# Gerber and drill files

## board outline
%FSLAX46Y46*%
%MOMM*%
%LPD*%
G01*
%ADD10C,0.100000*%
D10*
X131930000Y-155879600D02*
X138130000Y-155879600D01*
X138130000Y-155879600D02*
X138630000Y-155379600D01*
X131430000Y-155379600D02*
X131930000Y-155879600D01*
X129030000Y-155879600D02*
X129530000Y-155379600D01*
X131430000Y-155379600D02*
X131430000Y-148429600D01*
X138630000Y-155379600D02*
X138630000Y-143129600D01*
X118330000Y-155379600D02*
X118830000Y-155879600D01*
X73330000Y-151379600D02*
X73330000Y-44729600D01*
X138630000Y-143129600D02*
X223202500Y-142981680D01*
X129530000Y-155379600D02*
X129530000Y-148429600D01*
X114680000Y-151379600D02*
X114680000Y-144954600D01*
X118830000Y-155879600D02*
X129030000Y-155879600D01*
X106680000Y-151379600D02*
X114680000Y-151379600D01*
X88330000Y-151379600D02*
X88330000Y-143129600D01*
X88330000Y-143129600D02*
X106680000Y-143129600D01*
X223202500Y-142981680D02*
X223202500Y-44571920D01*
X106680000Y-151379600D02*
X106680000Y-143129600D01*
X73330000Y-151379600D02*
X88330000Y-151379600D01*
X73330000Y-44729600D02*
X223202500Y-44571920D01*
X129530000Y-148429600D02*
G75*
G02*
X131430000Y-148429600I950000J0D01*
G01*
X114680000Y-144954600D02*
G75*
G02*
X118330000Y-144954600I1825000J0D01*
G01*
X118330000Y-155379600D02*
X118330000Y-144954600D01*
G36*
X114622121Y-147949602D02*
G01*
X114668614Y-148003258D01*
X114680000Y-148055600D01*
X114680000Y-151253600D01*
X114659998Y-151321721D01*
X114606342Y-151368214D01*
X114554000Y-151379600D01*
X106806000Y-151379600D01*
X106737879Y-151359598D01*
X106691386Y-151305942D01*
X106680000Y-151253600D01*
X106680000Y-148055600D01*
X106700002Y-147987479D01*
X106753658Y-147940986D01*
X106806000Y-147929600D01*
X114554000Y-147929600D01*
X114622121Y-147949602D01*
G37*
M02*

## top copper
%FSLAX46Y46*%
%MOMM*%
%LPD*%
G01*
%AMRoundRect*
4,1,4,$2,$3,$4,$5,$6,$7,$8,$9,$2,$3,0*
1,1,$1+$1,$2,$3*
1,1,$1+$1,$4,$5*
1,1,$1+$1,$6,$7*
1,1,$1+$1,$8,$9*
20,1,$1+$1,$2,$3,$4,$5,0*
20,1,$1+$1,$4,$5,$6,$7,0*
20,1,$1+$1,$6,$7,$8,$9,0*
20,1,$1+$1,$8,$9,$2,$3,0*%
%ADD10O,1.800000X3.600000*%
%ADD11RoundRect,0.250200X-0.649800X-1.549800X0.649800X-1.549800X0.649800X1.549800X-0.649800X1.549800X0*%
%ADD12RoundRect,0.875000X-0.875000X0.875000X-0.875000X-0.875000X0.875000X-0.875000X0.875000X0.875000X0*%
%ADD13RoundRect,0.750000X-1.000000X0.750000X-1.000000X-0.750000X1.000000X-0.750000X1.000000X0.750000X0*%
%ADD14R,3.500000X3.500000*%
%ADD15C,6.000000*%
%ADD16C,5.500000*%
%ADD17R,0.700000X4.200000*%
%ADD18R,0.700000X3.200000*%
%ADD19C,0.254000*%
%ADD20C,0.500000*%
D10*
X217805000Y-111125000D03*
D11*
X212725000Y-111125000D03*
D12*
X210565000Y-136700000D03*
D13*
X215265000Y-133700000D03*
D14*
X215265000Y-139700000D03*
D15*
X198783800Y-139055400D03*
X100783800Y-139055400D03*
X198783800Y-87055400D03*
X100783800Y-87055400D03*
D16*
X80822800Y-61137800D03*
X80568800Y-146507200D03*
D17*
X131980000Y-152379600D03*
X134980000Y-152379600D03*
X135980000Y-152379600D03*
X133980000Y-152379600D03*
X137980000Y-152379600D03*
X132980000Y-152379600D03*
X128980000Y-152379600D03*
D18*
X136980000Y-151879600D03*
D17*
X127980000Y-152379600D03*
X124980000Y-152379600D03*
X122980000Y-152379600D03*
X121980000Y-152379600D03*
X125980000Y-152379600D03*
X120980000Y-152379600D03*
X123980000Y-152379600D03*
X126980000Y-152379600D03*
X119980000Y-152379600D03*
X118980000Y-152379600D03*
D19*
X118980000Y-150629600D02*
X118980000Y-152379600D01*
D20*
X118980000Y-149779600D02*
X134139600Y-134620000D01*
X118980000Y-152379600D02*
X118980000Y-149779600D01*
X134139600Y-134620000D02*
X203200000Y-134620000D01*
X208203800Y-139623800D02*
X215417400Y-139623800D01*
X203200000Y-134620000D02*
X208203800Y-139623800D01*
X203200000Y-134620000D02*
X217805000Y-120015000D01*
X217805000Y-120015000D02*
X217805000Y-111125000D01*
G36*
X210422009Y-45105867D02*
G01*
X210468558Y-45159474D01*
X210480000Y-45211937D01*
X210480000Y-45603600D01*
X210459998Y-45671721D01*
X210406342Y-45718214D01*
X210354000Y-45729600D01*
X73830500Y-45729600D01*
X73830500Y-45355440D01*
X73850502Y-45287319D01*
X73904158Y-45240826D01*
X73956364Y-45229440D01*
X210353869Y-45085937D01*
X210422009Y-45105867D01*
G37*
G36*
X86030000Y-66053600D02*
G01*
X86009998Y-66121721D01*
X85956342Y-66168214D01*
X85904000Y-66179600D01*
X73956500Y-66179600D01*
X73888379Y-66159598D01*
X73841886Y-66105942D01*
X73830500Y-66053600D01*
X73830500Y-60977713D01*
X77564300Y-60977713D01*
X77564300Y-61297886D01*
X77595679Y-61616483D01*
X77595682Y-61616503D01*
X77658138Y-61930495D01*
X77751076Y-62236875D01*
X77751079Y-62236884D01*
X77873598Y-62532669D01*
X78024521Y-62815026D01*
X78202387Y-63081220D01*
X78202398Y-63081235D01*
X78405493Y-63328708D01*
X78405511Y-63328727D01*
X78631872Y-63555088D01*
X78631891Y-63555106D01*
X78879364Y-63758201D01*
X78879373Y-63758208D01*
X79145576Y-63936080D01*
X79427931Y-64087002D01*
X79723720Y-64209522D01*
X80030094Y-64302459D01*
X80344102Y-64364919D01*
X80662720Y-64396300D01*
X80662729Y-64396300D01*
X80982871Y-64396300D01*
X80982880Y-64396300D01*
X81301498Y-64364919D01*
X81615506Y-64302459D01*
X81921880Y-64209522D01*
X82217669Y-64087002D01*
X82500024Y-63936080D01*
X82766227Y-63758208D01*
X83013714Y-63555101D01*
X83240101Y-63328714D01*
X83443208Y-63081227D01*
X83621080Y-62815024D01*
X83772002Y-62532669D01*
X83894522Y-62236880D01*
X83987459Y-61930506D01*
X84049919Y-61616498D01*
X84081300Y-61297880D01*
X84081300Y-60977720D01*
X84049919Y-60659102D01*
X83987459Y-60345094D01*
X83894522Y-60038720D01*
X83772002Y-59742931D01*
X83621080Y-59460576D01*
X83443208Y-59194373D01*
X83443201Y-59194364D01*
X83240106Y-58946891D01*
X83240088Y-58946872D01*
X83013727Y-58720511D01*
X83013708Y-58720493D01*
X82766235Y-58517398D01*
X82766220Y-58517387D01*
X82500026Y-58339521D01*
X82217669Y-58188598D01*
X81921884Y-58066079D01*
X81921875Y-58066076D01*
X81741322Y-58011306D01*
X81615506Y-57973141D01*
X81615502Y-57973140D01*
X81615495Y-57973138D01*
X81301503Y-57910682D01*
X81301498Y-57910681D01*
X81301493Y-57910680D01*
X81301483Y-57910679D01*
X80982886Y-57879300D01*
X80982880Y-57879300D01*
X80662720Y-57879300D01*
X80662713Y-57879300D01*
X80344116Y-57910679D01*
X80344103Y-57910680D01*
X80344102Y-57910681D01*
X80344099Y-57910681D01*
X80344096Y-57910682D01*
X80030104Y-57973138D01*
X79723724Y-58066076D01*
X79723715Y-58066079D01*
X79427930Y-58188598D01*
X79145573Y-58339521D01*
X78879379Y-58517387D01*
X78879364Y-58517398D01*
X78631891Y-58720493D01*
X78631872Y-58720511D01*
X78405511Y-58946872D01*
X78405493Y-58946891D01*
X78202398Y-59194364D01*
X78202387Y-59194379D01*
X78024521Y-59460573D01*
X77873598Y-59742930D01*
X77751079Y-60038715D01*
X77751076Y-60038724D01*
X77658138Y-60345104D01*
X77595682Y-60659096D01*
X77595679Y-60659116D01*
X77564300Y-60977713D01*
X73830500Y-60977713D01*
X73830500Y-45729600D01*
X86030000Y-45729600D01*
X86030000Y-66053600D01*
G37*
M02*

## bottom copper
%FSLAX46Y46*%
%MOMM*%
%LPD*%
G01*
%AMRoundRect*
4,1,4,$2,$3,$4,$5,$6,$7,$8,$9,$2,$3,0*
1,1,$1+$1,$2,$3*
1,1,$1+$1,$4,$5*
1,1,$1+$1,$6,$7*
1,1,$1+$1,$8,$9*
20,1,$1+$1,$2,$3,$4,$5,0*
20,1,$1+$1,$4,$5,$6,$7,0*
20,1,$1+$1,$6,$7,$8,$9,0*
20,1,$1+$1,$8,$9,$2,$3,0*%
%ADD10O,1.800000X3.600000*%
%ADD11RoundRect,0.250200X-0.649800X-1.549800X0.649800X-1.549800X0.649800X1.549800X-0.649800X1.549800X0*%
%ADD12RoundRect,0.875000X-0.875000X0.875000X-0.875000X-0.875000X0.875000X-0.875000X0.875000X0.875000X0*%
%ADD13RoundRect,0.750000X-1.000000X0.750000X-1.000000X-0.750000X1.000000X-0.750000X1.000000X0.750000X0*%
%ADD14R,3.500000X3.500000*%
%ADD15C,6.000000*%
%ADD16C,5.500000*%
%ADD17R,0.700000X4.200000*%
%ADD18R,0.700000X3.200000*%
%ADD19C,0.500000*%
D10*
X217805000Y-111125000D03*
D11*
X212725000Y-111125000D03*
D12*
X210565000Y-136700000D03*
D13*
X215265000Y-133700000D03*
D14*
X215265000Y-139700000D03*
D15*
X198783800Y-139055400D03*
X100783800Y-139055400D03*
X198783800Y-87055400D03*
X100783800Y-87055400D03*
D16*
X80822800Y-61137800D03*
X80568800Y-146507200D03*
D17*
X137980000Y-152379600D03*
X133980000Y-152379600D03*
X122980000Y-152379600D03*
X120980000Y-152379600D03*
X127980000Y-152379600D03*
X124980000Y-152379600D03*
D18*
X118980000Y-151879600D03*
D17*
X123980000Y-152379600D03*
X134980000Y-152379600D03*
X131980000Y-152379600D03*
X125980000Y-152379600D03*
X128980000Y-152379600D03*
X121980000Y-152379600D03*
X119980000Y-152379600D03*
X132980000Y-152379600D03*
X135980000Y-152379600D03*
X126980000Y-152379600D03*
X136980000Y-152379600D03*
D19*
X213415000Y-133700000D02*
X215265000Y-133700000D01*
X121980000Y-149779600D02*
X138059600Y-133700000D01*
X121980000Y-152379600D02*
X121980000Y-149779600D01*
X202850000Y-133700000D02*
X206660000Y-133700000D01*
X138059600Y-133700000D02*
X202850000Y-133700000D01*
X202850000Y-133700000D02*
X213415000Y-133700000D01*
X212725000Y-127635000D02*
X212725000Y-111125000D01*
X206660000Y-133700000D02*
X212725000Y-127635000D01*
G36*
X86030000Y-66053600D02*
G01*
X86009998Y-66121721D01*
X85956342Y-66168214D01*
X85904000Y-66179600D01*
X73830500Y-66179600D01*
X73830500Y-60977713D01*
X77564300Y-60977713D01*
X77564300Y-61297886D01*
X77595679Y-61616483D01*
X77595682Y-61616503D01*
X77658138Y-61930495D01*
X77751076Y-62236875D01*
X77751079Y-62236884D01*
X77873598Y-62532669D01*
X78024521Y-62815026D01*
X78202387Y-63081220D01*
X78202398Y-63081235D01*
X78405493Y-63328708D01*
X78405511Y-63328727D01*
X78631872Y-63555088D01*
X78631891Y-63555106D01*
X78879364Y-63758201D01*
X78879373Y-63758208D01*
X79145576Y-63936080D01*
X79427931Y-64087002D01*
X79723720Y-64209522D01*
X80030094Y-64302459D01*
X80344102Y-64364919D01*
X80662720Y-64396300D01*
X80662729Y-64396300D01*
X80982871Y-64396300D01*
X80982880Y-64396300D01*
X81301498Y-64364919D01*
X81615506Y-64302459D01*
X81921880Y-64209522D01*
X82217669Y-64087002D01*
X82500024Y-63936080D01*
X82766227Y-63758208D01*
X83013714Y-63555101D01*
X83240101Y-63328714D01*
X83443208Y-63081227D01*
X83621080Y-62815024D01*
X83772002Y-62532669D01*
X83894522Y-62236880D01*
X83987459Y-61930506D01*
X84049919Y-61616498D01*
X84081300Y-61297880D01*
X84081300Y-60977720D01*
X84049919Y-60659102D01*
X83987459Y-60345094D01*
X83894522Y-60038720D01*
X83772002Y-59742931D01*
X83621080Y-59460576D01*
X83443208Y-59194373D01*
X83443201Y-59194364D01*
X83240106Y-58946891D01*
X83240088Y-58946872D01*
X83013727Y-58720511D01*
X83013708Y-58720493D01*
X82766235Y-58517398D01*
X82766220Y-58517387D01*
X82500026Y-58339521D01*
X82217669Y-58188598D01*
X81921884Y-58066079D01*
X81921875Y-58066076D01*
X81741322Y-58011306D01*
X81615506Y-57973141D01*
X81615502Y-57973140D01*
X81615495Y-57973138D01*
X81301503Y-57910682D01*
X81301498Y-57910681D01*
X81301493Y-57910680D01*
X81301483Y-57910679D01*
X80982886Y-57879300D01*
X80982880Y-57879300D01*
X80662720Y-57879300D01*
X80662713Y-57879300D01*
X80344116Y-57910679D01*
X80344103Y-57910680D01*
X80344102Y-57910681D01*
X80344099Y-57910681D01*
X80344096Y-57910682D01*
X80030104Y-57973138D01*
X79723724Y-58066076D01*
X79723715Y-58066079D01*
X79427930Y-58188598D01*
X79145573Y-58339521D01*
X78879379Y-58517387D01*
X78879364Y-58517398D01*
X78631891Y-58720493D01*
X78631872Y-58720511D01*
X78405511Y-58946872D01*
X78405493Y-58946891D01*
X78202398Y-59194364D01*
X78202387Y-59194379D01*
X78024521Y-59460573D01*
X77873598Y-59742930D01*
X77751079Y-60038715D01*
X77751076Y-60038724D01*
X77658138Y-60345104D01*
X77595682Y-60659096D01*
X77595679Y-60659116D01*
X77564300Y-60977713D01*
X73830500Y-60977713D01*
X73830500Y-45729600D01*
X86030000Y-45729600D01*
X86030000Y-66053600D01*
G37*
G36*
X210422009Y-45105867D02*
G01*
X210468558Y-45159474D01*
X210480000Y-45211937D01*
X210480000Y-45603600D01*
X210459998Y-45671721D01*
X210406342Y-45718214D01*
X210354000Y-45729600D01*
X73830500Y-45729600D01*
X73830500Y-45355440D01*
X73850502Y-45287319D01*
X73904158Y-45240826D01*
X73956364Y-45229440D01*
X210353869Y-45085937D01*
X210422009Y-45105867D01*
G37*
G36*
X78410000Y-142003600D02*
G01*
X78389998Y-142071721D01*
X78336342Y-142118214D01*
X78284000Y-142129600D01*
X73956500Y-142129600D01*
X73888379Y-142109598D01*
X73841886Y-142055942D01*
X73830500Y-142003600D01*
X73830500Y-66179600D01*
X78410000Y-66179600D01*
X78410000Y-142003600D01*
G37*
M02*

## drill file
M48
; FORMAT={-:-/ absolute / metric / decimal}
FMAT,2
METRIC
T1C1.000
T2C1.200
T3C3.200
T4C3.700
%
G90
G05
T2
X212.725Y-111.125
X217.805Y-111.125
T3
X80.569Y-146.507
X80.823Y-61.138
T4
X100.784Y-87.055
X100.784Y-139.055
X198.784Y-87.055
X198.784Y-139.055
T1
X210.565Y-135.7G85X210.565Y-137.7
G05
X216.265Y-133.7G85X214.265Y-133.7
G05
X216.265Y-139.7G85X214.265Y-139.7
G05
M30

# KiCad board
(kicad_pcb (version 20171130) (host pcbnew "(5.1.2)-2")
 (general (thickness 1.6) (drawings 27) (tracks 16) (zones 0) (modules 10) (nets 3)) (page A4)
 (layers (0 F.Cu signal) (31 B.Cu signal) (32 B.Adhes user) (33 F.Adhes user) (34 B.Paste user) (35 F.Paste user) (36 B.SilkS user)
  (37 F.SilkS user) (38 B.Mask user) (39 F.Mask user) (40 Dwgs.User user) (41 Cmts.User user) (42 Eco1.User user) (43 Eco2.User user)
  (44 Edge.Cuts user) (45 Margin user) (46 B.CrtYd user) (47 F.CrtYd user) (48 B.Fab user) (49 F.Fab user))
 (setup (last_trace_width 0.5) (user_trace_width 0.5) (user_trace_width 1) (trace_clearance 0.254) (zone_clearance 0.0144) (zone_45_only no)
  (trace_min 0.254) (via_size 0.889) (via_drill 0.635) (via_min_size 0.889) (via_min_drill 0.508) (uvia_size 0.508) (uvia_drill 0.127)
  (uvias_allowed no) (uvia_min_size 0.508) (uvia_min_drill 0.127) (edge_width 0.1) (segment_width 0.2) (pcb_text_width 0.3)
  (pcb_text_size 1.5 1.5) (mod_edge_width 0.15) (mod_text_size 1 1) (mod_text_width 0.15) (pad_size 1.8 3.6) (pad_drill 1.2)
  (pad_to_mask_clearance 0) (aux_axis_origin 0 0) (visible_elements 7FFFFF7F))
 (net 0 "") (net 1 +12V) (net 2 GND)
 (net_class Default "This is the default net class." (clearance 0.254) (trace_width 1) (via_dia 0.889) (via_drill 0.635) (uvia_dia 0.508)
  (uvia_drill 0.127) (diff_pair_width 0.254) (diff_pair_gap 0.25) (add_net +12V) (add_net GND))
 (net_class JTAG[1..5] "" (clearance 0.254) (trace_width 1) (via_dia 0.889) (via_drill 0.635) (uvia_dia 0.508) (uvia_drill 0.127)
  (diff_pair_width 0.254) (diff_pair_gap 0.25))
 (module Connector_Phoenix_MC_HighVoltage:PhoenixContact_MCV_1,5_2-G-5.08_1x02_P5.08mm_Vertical (layer F.Cu) (at 212.725 111.125)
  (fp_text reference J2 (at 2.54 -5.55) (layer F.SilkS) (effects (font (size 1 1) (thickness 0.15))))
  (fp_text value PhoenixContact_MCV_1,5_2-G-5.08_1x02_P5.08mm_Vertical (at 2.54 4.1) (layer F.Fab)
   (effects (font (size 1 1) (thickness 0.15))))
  (pad 2 thru_hole oval (at 5.08 0) (size 1.8 3.6) (drill 1.2) (layers *.Cu *.Mask) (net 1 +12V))
  (pad 1 thru_hole roundrect (at 0 0) (size 1.8 3.6) (drill 1.2) (layers *.Cu *.Mask) (roundrect_rratio 0.139) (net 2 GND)))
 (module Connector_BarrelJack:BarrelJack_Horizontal (layer F.Cu) (at 215.265 139.7 270)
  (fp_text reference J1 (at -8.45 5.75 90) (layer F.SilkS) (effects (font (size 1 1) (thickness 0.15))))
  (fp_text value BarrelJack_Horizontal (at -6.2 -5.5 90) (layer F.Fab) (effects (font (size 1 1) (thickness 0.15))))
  (pad 3 thru_hole roundrect (at -3 4.7 270) (size 3.5 3.5) (drill oval 3 1) (layers *.Cu *.Mask) (roundrect_rratio 0.25))
  (pad 2 thru_hole roundrect (at -6 0 270) (size 3 3.5) (drill oval 1 3) (layers *.Cu *.Mask) (roundrect_rratio 0.25) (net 2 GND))
  (pad 1 thru_hole rect (at 0 0 270) (size 3.5 3.5) (drill oval 1 3) (layers *.Cu *.Mask) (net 1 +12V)))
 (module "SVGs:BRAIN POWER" (layer B.Cu) (at 155.575 97.79 180)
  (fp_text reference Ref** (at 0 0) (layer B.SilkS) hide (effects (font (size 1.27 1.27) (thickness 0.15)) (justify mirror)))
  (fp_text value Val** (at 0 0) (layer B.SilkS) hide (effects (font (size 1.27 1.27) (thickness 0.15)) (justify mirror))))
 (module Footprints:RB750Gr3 (layer F.Cu) (at 149.7838 113.0554)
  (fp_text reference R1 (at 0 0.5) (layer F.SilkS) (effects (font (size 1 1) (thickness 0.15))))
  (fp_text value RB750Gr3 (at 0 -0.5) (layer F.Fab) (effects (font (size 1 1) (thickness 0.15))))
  (pad 4 thru_hole circle (at 49 26) (size 6 6) (drill 3.7) (layers *.Cu *.Mask))
  (pad 3 thru_hole circle (at -49 26) (size 6 6) (drill 3.7) (layers *.Cu *.Mask))
  (pad 2 thru_hole circle (at 49 -26) (size 6 6) (drill 3.7) (layers *.Cu *.Mask))
  (pad 1 thru_hole circle (at -49 -26) (size 6 6) (drill 3.7) (layers *.Cu *.Mask)))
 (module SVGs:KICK (layer F.Cu) (at 148.9456 53.4416)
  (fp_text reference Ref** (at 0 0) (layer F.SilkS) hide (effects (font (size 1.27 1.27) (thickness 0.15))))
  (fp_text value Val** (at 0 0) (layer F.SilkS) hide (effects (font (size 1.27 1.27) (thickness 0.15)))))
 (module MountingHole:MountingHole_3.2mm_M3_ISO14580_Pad (layer F.Cu) (at 80.8228 61.1378)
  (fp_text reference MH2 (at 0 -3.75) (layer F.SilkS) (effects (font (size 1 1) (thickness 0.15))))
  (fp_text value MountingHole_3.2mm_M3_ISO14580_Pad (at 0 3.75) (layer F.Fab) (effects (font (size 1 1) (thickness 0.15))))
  (pad 1 thru_hole circle (at 0 0) (size 5.5 5.5) (drill 3.2) (layers *.Cu *.Mask)))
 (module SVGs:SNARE (layer B.Cu) (at 148.1582 53.5178 180)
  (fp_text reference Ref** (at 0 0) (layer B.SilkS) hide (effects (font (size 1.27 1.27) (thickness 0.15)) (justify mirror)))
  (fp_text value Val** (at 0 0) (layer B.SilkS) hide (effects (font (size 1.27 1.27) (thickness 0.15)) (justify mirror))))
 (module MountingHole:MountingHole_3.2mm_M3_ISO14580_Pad (layer F.Cu) (at 80.5688 146.5072)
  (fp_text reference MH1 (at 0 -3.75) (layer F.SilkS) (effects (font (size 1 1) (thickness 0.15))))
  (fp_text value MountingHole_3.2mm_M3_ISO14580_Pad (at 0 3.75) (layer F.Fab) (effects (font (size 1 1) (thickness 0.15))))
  (pad 1 thru_hole circle (at 0 0) (size 5.5 5.5) (drill 3.2) (layers *.Cu *.Mask)))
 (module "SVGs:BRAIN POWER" (layer F.Cu) (at 220.98 -163.83)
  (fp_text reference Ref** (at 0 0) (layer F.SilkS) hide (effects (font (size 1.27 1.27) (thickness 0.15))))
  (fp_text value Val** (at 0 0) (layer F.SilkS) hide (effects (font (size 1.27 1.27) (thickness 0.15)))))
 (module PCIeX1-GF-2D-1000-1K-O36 (layer F.Cu) (at 128.48 152.3796)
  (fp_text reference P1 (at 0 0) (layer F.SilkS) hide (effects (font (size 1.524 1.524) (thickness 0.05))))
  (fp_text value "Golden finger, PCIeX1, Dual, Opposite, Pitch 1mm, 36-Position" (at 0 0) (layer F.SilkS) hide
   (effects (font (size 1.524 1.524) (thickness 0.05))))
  (pad B12 smd rect (at 3.5 0) (size 0.7 4.2) (layers F.Cu F.Paste F.Mask))
  (pad B15 smd rect (at 6.5 0) (size 0.7 4.2) (layers F.Cu F.Paste F.Mask))
  (pad B16 smd rect (at 7.5 0) (size 0.7 4.2) (layers F.Cu F.Paste F.Mask))
  (pad B14 smd rect (at 5.5 0) (size 0.7 4.2) (layers F.Cu F.Paste F.Mask))
  (pad B18 smd rect (at 9.5 0) (size 0.7 4.2) (layers F.Cu F.Paste F.Mask))
  (pad B13 smd rect (at 4.5 0) (size 0.7 4.2) (layers F.Cu F.Paste F.Mask))
  (pad B11 smd rect (at 0.5 0) (size 0.7 4.2) (layers F.Cu F.Paste F.Mask))
  (pad B17 smd rect (at 8.5 -0.5) (size 0.7 3.2) (layers F.Cu F.Paste F.Mask))
  (pad B10 smd rect (at -0.5 0) (size 0.7 4.2) (layers F.Cu F.Paste F.Mask))
  (pad B7 smd rect (at -3.5 0) (size 0.7 4.2) (layers F.Cu F.Paste F.Mask))
  (pad B5 smd rect (at -5.5 0) (size 0.7 4.2) (layers F.Cu F.Paste F.Mask))
  (pad B4 smd rect (at -6.5 0) (size 0.7 4.2) (layers F.Cu F.Paste F.Mask))
  (pad B8 smd rect (at -2.5 0) (size 0.7 4.2) (layers F.Cu F.Paste F.Mask))
  (pad B3 smd rect (at -7.5 0) (size 0.7 4.2) (layers F.Cu F.Paste F.Mask))
  (pad B6 smd rect (at -4.5 0) (size 0.7 4.2) (layers F.Cu F.Paste F.Mask))
  (pad B9 smd rect (at -1.5 0) (size 0.7 4.2) (layers F.Cu F.Paste F.Mask))
  (pad B2 smd rect (at -8.5 0) (size 0.7 4.2) (layers F.Cu F.Paste F.Mask))
  (pad B1 smd rect (at -9.5 0) (size 0.7 4.2) (layers F.Cu F.Paste F.Mask) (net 1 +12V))
  (pad A18 smd rect (at 9.5 0) (size 0.7 4.2) (layers B.Cu B.Paste B.Mask))
  (pad A14 smd rect (at 5.5 0) (size 0.7 4.2) (layers B.Cu B.Paste B.Mask))
  (pad A5 smd rect (at -5.5 0) (size 0.7 4.2) (layers B.Cu B.Paste B.Mask))
  (pad A3 smd rect (at -7.5 0) (size 0.7 4.2) (layers B.Cu B.Paste B.Mask))
  (pad A10 smd rect (at -0.5 0) (size 0.7 4.2) (layers B.Cu B.Paste B.Mask))
  (pad A7 smd rect (at -3.5 0) (size 0.7 4.2) (layers B.Cu B.Paste B.Mask))
  (pad A1 smd rect (at -9.5 -0.5) (size 0.7 3.2) (layers B.Cu B.Paste B.Mask))
  (pad A6 smd rect (at -4.5 0) (size 0.7 4.2) (layers B.Cu B.Paste B.Mask))
  (pad A15 smd rect (at 6.5 0) (size 0.7 4.2) (layers B.Cu B.Paste B.Mask))
  (pad A12 smd rect (at 3.5 0) (size 0.7 4.2) (layers B.Cu B.Paste B.Mask))
  (pad A8 smd rect (at -2.5 0) (size 0.7 4.2) (layers B.Cu B.Paste B.Mask))
  (pad A11 smd rect (at 0.5 0) (size 0.7 4.2) (layers B.Cu B.Paste B.Mask))
  (pad A4 smd rect (at -6.5 0) (size 0.7 4.2) (layers B.Cu B.Paste B.Mask) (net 2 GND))
  (pad A2 smd rect (at -8.5 0) (size 0.7 4.2) (layers B.Cu B.Paste B.Mask))
  (pad A13 smd rect (at 4.5 0) (size 0.7 4.2) (layers B.Cu B.Paste B.Mask))
  (pad A16 smd rect (at 7.5 0) (size 0.7 4.2) (layers B.Cu B.Paste B.Mask))
  (pad A9 smd rect (at -1.5 0) (size 0.7 4.2) (layers B.Cu B.Paste B.Mask))
  (pad A17 smd rect (at 8.5 0) (size 0.7 4.2) (layers B.Cu B.Paste B.Mask)))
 (gr_line (start 131.93 155.8796) (end 138.13 155.8796) (layer Edge.Cuts) (width 0.1))
 (gr_line (start 138.13 155.8796) (end 138.63 155.3796) (layer Edge.Cuts) (width 0.1))
 (gr_line (start 131.43 155.3796) (end 131.93 155.8796) (layer Edge.Cuts) (width 0.1))
 (gr_line (start 129.03 155.8796) (end 129.53 155.3796) (layer Edge.Cuts) (width 0.1))
 (gr_line (start 131.43 155.3796) (end 131.43 148.4296) (layer Edge.Cuts) (width 0.1))
 (gr_line (start 138.63 155.3796) (end 138.63 143.1296) (layer Edge.Cuts) (width 0.1))
 (gr_line (start 118.33 155.3796) (end 118.83 155.8796) (layer Edge.Cuts) (width 0.1))
 (gr_line (start 73.33 151.3796) (end 73.33 44.7296) (layer Edge.Cuts) (width 0.1))
 (gr_line (start 138.63 143.1296) (end 223.2025 142.98168) (layer Edge.Cuts) (width 0.1))
 (gr_line (start 129.53 155.3796) (end 129.53 148.4296) (layer Edge.Cuts) (width 0.1))
 (gr_line (start 114.68 151.3796) (end 114.68 144.9546) (layer Edge.Cuts) (width 0.1))
 (gr_line (start 118.83 155.8796) (end 129.03 155.8796) (layer Edge.Cuts) (width 0.1))
 (gr_line (start 106.68 151.3796) (end 114.68 151.3796) (layer Edge.Cuts) (width 0.1))
 (gr_line (start 88.33 151.3796) (end 88.33 143.1296) (layer Edge.Cuts) (width 0.1))
 (gr_line (start 88.33 143.1296) (end 106.68 143.1296) (layer Edge.Cuts) (width 0.1))
 (gr_line (start 223.2025 142.98168) (end 223.2025 44.57192) (layer Edge.Cuts) (width 0.1))
 (gr_line (start 106.68 151.3796) (end 106.68 143.1296) (layer Edge.Cuts) (width 0.1))
 (gr_line (start 73.33 151.3796) (end 88.33 151.3796) (layer Edge.Cuts) (width 0.1))
 (gr_line (start 73.33 44.7296) (end 223.2025 44.57192) (layer Edge.Cuts) (width 0.1))
 (gr_arc (start 130.48 148.4296) (end 131.43 148.4296) (angle -180) (layer Edge.Cuts) (width 0.1))
 (gr_arc (start 116.505 144.9546) (end 118.33 144.9546) (angle -180) (layer Edge.Cuts) (width 0.1))
 (gr_line (start 118.33 155.3796) (end 118.33 144.9546) (layer Edge.Cuts) (width 0.1))
 (segment (start 213.415 133.7) (end 215.265 133.7) (width 0.5) (layer B.Cu) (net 2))
 (segment (start 121.98 149.7796) (end 138.0596 133.7) (width 0.5) (layer B.Cu) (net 2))
 (segment (start 121.98 152.3796) (end 121.98 149.7796) (width 0.5) (layer B.Cu) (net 2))
 (segment (start 202.85 133.7) (end 206.66 133.7) (width 0.5) (layer B.Cu) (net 2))
 (segment (start 138.0596 133.7) (end 202.85 133.7) (width 0.5) (layer B.Cu) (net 2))
 (segment (start 202.85 133.7) (end 213.415 133.7) (width 0.5) (layer B.Cu) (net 2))
 (segment (start 212.725 127.635) (end 212.725 111.125) (width 0.5) (layer B.Cu) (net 2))
 (segment (start 206.66 133.7) (end 212.725 127.635) (width 0.5) (layer B.Cu) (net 2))
 (segment (start 118.98 150.6296) (end 118.98 152.3796) (width 0.254) (layer F.Cu) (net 1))
 (segment (start 118.98 149.7796) (end 134.1396 134.62) (width 0.5) (layer F.Cu) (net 1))
 (segment (start 118.98 152.3796) (end 118.98 149.7796) (width 0.5) (layer F.Cu) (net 1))
 (segment (start 134.1396 134.62) (end 203.2 134.62) (width 0.5) (layer F.Cu) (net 1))
 (segment (start 208.2038 139.6238) (end 215.4174 139.6238) (width 0.5) (layer F.Cu) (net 1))
 (segment (start 203.2 134.62) (end 208.2038 139.6238) (width 0.5) (layer F.Cu) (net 1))
 (segment (start 203.2 134.62) (end 217.805 120.015) (width 0.5) (layer F.Cu) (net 1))
 (segment (start 217.805 120.015) (end 217.805 111.125) (width 0.5) (layer F.Cu) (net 1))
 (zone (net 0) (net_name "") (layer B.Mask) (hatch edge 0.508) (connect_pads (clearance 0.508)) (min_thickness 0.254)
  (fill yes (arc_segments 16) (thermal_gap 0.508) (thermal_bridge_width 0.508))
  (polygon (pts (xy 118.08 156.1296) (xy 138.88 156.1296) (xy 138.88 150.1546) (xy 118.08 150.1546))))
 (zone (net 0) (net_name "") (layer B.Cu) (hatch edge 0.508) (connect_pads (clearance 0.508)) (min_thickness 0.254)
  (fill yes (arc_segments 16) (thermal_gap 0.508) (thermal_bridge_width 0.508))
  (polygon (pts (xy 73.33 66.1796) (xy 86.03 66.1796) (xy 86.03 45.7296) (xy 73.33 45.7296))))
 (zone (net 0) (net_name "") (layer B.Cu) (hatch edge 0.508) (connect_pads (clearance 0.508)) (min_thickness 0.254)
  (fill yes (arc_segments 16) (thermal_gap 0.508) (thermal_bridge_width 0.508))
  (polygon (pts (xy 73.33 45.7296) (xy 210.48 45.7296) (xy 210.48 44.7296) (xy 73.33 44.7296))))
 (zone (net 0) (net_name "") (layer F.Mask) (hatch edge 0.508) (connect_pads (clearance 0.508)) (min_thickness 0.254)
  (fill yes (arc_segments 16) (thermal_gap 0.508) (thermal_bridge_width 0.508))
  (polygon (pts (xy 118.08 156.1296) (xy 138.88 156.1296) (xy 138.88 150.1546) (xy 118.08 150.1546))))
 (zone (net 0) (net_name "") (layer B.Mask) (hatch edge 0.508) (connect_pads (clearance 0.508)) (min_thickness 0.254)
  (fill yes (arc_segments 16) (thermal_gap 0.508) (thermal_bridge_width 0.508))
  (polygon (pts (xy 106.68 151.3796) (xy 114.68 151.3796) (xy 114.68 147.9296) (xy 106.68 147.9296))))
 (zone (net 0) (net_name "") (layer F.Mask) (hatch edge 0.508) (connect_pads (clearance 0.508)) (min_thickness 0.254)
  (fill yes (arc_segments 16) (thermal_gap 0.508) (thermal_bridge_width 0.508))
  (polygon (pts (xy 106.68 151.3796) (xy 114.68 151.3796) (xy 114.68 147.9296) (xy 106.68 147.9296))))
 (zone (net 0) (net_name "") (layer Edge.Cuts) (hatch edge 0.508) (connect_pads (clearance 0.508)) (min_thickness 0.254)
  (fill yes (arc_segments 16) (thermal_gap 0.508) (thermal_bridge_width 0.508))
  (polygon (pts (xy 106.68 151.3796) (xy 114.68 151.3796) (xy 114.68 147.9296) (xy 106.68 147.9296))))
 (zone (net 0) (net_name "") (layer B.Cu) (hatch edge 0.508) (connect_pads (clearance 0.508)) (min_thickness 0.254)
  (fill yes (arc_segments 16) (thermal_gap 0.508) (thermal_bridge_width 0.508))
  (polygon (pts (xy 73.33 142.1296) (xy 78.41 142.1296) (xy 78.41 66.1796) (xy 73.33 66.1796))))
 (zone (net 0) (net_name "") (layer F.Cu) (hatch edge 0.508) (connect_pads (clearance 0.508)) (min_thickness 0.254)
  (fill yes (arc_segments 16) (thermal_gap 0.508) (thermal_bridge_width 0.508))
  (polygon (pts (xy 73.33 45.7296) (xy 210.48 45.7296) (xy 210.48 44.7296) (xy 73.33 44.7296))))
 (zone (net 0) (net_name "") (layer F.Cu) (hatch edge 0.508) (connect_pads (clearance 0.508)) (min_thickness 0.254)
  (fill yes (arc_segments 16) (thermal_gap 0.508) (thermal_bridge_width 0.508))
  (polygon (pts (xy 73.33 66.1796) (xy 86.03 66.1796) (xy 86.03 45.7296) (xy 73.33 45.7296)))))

